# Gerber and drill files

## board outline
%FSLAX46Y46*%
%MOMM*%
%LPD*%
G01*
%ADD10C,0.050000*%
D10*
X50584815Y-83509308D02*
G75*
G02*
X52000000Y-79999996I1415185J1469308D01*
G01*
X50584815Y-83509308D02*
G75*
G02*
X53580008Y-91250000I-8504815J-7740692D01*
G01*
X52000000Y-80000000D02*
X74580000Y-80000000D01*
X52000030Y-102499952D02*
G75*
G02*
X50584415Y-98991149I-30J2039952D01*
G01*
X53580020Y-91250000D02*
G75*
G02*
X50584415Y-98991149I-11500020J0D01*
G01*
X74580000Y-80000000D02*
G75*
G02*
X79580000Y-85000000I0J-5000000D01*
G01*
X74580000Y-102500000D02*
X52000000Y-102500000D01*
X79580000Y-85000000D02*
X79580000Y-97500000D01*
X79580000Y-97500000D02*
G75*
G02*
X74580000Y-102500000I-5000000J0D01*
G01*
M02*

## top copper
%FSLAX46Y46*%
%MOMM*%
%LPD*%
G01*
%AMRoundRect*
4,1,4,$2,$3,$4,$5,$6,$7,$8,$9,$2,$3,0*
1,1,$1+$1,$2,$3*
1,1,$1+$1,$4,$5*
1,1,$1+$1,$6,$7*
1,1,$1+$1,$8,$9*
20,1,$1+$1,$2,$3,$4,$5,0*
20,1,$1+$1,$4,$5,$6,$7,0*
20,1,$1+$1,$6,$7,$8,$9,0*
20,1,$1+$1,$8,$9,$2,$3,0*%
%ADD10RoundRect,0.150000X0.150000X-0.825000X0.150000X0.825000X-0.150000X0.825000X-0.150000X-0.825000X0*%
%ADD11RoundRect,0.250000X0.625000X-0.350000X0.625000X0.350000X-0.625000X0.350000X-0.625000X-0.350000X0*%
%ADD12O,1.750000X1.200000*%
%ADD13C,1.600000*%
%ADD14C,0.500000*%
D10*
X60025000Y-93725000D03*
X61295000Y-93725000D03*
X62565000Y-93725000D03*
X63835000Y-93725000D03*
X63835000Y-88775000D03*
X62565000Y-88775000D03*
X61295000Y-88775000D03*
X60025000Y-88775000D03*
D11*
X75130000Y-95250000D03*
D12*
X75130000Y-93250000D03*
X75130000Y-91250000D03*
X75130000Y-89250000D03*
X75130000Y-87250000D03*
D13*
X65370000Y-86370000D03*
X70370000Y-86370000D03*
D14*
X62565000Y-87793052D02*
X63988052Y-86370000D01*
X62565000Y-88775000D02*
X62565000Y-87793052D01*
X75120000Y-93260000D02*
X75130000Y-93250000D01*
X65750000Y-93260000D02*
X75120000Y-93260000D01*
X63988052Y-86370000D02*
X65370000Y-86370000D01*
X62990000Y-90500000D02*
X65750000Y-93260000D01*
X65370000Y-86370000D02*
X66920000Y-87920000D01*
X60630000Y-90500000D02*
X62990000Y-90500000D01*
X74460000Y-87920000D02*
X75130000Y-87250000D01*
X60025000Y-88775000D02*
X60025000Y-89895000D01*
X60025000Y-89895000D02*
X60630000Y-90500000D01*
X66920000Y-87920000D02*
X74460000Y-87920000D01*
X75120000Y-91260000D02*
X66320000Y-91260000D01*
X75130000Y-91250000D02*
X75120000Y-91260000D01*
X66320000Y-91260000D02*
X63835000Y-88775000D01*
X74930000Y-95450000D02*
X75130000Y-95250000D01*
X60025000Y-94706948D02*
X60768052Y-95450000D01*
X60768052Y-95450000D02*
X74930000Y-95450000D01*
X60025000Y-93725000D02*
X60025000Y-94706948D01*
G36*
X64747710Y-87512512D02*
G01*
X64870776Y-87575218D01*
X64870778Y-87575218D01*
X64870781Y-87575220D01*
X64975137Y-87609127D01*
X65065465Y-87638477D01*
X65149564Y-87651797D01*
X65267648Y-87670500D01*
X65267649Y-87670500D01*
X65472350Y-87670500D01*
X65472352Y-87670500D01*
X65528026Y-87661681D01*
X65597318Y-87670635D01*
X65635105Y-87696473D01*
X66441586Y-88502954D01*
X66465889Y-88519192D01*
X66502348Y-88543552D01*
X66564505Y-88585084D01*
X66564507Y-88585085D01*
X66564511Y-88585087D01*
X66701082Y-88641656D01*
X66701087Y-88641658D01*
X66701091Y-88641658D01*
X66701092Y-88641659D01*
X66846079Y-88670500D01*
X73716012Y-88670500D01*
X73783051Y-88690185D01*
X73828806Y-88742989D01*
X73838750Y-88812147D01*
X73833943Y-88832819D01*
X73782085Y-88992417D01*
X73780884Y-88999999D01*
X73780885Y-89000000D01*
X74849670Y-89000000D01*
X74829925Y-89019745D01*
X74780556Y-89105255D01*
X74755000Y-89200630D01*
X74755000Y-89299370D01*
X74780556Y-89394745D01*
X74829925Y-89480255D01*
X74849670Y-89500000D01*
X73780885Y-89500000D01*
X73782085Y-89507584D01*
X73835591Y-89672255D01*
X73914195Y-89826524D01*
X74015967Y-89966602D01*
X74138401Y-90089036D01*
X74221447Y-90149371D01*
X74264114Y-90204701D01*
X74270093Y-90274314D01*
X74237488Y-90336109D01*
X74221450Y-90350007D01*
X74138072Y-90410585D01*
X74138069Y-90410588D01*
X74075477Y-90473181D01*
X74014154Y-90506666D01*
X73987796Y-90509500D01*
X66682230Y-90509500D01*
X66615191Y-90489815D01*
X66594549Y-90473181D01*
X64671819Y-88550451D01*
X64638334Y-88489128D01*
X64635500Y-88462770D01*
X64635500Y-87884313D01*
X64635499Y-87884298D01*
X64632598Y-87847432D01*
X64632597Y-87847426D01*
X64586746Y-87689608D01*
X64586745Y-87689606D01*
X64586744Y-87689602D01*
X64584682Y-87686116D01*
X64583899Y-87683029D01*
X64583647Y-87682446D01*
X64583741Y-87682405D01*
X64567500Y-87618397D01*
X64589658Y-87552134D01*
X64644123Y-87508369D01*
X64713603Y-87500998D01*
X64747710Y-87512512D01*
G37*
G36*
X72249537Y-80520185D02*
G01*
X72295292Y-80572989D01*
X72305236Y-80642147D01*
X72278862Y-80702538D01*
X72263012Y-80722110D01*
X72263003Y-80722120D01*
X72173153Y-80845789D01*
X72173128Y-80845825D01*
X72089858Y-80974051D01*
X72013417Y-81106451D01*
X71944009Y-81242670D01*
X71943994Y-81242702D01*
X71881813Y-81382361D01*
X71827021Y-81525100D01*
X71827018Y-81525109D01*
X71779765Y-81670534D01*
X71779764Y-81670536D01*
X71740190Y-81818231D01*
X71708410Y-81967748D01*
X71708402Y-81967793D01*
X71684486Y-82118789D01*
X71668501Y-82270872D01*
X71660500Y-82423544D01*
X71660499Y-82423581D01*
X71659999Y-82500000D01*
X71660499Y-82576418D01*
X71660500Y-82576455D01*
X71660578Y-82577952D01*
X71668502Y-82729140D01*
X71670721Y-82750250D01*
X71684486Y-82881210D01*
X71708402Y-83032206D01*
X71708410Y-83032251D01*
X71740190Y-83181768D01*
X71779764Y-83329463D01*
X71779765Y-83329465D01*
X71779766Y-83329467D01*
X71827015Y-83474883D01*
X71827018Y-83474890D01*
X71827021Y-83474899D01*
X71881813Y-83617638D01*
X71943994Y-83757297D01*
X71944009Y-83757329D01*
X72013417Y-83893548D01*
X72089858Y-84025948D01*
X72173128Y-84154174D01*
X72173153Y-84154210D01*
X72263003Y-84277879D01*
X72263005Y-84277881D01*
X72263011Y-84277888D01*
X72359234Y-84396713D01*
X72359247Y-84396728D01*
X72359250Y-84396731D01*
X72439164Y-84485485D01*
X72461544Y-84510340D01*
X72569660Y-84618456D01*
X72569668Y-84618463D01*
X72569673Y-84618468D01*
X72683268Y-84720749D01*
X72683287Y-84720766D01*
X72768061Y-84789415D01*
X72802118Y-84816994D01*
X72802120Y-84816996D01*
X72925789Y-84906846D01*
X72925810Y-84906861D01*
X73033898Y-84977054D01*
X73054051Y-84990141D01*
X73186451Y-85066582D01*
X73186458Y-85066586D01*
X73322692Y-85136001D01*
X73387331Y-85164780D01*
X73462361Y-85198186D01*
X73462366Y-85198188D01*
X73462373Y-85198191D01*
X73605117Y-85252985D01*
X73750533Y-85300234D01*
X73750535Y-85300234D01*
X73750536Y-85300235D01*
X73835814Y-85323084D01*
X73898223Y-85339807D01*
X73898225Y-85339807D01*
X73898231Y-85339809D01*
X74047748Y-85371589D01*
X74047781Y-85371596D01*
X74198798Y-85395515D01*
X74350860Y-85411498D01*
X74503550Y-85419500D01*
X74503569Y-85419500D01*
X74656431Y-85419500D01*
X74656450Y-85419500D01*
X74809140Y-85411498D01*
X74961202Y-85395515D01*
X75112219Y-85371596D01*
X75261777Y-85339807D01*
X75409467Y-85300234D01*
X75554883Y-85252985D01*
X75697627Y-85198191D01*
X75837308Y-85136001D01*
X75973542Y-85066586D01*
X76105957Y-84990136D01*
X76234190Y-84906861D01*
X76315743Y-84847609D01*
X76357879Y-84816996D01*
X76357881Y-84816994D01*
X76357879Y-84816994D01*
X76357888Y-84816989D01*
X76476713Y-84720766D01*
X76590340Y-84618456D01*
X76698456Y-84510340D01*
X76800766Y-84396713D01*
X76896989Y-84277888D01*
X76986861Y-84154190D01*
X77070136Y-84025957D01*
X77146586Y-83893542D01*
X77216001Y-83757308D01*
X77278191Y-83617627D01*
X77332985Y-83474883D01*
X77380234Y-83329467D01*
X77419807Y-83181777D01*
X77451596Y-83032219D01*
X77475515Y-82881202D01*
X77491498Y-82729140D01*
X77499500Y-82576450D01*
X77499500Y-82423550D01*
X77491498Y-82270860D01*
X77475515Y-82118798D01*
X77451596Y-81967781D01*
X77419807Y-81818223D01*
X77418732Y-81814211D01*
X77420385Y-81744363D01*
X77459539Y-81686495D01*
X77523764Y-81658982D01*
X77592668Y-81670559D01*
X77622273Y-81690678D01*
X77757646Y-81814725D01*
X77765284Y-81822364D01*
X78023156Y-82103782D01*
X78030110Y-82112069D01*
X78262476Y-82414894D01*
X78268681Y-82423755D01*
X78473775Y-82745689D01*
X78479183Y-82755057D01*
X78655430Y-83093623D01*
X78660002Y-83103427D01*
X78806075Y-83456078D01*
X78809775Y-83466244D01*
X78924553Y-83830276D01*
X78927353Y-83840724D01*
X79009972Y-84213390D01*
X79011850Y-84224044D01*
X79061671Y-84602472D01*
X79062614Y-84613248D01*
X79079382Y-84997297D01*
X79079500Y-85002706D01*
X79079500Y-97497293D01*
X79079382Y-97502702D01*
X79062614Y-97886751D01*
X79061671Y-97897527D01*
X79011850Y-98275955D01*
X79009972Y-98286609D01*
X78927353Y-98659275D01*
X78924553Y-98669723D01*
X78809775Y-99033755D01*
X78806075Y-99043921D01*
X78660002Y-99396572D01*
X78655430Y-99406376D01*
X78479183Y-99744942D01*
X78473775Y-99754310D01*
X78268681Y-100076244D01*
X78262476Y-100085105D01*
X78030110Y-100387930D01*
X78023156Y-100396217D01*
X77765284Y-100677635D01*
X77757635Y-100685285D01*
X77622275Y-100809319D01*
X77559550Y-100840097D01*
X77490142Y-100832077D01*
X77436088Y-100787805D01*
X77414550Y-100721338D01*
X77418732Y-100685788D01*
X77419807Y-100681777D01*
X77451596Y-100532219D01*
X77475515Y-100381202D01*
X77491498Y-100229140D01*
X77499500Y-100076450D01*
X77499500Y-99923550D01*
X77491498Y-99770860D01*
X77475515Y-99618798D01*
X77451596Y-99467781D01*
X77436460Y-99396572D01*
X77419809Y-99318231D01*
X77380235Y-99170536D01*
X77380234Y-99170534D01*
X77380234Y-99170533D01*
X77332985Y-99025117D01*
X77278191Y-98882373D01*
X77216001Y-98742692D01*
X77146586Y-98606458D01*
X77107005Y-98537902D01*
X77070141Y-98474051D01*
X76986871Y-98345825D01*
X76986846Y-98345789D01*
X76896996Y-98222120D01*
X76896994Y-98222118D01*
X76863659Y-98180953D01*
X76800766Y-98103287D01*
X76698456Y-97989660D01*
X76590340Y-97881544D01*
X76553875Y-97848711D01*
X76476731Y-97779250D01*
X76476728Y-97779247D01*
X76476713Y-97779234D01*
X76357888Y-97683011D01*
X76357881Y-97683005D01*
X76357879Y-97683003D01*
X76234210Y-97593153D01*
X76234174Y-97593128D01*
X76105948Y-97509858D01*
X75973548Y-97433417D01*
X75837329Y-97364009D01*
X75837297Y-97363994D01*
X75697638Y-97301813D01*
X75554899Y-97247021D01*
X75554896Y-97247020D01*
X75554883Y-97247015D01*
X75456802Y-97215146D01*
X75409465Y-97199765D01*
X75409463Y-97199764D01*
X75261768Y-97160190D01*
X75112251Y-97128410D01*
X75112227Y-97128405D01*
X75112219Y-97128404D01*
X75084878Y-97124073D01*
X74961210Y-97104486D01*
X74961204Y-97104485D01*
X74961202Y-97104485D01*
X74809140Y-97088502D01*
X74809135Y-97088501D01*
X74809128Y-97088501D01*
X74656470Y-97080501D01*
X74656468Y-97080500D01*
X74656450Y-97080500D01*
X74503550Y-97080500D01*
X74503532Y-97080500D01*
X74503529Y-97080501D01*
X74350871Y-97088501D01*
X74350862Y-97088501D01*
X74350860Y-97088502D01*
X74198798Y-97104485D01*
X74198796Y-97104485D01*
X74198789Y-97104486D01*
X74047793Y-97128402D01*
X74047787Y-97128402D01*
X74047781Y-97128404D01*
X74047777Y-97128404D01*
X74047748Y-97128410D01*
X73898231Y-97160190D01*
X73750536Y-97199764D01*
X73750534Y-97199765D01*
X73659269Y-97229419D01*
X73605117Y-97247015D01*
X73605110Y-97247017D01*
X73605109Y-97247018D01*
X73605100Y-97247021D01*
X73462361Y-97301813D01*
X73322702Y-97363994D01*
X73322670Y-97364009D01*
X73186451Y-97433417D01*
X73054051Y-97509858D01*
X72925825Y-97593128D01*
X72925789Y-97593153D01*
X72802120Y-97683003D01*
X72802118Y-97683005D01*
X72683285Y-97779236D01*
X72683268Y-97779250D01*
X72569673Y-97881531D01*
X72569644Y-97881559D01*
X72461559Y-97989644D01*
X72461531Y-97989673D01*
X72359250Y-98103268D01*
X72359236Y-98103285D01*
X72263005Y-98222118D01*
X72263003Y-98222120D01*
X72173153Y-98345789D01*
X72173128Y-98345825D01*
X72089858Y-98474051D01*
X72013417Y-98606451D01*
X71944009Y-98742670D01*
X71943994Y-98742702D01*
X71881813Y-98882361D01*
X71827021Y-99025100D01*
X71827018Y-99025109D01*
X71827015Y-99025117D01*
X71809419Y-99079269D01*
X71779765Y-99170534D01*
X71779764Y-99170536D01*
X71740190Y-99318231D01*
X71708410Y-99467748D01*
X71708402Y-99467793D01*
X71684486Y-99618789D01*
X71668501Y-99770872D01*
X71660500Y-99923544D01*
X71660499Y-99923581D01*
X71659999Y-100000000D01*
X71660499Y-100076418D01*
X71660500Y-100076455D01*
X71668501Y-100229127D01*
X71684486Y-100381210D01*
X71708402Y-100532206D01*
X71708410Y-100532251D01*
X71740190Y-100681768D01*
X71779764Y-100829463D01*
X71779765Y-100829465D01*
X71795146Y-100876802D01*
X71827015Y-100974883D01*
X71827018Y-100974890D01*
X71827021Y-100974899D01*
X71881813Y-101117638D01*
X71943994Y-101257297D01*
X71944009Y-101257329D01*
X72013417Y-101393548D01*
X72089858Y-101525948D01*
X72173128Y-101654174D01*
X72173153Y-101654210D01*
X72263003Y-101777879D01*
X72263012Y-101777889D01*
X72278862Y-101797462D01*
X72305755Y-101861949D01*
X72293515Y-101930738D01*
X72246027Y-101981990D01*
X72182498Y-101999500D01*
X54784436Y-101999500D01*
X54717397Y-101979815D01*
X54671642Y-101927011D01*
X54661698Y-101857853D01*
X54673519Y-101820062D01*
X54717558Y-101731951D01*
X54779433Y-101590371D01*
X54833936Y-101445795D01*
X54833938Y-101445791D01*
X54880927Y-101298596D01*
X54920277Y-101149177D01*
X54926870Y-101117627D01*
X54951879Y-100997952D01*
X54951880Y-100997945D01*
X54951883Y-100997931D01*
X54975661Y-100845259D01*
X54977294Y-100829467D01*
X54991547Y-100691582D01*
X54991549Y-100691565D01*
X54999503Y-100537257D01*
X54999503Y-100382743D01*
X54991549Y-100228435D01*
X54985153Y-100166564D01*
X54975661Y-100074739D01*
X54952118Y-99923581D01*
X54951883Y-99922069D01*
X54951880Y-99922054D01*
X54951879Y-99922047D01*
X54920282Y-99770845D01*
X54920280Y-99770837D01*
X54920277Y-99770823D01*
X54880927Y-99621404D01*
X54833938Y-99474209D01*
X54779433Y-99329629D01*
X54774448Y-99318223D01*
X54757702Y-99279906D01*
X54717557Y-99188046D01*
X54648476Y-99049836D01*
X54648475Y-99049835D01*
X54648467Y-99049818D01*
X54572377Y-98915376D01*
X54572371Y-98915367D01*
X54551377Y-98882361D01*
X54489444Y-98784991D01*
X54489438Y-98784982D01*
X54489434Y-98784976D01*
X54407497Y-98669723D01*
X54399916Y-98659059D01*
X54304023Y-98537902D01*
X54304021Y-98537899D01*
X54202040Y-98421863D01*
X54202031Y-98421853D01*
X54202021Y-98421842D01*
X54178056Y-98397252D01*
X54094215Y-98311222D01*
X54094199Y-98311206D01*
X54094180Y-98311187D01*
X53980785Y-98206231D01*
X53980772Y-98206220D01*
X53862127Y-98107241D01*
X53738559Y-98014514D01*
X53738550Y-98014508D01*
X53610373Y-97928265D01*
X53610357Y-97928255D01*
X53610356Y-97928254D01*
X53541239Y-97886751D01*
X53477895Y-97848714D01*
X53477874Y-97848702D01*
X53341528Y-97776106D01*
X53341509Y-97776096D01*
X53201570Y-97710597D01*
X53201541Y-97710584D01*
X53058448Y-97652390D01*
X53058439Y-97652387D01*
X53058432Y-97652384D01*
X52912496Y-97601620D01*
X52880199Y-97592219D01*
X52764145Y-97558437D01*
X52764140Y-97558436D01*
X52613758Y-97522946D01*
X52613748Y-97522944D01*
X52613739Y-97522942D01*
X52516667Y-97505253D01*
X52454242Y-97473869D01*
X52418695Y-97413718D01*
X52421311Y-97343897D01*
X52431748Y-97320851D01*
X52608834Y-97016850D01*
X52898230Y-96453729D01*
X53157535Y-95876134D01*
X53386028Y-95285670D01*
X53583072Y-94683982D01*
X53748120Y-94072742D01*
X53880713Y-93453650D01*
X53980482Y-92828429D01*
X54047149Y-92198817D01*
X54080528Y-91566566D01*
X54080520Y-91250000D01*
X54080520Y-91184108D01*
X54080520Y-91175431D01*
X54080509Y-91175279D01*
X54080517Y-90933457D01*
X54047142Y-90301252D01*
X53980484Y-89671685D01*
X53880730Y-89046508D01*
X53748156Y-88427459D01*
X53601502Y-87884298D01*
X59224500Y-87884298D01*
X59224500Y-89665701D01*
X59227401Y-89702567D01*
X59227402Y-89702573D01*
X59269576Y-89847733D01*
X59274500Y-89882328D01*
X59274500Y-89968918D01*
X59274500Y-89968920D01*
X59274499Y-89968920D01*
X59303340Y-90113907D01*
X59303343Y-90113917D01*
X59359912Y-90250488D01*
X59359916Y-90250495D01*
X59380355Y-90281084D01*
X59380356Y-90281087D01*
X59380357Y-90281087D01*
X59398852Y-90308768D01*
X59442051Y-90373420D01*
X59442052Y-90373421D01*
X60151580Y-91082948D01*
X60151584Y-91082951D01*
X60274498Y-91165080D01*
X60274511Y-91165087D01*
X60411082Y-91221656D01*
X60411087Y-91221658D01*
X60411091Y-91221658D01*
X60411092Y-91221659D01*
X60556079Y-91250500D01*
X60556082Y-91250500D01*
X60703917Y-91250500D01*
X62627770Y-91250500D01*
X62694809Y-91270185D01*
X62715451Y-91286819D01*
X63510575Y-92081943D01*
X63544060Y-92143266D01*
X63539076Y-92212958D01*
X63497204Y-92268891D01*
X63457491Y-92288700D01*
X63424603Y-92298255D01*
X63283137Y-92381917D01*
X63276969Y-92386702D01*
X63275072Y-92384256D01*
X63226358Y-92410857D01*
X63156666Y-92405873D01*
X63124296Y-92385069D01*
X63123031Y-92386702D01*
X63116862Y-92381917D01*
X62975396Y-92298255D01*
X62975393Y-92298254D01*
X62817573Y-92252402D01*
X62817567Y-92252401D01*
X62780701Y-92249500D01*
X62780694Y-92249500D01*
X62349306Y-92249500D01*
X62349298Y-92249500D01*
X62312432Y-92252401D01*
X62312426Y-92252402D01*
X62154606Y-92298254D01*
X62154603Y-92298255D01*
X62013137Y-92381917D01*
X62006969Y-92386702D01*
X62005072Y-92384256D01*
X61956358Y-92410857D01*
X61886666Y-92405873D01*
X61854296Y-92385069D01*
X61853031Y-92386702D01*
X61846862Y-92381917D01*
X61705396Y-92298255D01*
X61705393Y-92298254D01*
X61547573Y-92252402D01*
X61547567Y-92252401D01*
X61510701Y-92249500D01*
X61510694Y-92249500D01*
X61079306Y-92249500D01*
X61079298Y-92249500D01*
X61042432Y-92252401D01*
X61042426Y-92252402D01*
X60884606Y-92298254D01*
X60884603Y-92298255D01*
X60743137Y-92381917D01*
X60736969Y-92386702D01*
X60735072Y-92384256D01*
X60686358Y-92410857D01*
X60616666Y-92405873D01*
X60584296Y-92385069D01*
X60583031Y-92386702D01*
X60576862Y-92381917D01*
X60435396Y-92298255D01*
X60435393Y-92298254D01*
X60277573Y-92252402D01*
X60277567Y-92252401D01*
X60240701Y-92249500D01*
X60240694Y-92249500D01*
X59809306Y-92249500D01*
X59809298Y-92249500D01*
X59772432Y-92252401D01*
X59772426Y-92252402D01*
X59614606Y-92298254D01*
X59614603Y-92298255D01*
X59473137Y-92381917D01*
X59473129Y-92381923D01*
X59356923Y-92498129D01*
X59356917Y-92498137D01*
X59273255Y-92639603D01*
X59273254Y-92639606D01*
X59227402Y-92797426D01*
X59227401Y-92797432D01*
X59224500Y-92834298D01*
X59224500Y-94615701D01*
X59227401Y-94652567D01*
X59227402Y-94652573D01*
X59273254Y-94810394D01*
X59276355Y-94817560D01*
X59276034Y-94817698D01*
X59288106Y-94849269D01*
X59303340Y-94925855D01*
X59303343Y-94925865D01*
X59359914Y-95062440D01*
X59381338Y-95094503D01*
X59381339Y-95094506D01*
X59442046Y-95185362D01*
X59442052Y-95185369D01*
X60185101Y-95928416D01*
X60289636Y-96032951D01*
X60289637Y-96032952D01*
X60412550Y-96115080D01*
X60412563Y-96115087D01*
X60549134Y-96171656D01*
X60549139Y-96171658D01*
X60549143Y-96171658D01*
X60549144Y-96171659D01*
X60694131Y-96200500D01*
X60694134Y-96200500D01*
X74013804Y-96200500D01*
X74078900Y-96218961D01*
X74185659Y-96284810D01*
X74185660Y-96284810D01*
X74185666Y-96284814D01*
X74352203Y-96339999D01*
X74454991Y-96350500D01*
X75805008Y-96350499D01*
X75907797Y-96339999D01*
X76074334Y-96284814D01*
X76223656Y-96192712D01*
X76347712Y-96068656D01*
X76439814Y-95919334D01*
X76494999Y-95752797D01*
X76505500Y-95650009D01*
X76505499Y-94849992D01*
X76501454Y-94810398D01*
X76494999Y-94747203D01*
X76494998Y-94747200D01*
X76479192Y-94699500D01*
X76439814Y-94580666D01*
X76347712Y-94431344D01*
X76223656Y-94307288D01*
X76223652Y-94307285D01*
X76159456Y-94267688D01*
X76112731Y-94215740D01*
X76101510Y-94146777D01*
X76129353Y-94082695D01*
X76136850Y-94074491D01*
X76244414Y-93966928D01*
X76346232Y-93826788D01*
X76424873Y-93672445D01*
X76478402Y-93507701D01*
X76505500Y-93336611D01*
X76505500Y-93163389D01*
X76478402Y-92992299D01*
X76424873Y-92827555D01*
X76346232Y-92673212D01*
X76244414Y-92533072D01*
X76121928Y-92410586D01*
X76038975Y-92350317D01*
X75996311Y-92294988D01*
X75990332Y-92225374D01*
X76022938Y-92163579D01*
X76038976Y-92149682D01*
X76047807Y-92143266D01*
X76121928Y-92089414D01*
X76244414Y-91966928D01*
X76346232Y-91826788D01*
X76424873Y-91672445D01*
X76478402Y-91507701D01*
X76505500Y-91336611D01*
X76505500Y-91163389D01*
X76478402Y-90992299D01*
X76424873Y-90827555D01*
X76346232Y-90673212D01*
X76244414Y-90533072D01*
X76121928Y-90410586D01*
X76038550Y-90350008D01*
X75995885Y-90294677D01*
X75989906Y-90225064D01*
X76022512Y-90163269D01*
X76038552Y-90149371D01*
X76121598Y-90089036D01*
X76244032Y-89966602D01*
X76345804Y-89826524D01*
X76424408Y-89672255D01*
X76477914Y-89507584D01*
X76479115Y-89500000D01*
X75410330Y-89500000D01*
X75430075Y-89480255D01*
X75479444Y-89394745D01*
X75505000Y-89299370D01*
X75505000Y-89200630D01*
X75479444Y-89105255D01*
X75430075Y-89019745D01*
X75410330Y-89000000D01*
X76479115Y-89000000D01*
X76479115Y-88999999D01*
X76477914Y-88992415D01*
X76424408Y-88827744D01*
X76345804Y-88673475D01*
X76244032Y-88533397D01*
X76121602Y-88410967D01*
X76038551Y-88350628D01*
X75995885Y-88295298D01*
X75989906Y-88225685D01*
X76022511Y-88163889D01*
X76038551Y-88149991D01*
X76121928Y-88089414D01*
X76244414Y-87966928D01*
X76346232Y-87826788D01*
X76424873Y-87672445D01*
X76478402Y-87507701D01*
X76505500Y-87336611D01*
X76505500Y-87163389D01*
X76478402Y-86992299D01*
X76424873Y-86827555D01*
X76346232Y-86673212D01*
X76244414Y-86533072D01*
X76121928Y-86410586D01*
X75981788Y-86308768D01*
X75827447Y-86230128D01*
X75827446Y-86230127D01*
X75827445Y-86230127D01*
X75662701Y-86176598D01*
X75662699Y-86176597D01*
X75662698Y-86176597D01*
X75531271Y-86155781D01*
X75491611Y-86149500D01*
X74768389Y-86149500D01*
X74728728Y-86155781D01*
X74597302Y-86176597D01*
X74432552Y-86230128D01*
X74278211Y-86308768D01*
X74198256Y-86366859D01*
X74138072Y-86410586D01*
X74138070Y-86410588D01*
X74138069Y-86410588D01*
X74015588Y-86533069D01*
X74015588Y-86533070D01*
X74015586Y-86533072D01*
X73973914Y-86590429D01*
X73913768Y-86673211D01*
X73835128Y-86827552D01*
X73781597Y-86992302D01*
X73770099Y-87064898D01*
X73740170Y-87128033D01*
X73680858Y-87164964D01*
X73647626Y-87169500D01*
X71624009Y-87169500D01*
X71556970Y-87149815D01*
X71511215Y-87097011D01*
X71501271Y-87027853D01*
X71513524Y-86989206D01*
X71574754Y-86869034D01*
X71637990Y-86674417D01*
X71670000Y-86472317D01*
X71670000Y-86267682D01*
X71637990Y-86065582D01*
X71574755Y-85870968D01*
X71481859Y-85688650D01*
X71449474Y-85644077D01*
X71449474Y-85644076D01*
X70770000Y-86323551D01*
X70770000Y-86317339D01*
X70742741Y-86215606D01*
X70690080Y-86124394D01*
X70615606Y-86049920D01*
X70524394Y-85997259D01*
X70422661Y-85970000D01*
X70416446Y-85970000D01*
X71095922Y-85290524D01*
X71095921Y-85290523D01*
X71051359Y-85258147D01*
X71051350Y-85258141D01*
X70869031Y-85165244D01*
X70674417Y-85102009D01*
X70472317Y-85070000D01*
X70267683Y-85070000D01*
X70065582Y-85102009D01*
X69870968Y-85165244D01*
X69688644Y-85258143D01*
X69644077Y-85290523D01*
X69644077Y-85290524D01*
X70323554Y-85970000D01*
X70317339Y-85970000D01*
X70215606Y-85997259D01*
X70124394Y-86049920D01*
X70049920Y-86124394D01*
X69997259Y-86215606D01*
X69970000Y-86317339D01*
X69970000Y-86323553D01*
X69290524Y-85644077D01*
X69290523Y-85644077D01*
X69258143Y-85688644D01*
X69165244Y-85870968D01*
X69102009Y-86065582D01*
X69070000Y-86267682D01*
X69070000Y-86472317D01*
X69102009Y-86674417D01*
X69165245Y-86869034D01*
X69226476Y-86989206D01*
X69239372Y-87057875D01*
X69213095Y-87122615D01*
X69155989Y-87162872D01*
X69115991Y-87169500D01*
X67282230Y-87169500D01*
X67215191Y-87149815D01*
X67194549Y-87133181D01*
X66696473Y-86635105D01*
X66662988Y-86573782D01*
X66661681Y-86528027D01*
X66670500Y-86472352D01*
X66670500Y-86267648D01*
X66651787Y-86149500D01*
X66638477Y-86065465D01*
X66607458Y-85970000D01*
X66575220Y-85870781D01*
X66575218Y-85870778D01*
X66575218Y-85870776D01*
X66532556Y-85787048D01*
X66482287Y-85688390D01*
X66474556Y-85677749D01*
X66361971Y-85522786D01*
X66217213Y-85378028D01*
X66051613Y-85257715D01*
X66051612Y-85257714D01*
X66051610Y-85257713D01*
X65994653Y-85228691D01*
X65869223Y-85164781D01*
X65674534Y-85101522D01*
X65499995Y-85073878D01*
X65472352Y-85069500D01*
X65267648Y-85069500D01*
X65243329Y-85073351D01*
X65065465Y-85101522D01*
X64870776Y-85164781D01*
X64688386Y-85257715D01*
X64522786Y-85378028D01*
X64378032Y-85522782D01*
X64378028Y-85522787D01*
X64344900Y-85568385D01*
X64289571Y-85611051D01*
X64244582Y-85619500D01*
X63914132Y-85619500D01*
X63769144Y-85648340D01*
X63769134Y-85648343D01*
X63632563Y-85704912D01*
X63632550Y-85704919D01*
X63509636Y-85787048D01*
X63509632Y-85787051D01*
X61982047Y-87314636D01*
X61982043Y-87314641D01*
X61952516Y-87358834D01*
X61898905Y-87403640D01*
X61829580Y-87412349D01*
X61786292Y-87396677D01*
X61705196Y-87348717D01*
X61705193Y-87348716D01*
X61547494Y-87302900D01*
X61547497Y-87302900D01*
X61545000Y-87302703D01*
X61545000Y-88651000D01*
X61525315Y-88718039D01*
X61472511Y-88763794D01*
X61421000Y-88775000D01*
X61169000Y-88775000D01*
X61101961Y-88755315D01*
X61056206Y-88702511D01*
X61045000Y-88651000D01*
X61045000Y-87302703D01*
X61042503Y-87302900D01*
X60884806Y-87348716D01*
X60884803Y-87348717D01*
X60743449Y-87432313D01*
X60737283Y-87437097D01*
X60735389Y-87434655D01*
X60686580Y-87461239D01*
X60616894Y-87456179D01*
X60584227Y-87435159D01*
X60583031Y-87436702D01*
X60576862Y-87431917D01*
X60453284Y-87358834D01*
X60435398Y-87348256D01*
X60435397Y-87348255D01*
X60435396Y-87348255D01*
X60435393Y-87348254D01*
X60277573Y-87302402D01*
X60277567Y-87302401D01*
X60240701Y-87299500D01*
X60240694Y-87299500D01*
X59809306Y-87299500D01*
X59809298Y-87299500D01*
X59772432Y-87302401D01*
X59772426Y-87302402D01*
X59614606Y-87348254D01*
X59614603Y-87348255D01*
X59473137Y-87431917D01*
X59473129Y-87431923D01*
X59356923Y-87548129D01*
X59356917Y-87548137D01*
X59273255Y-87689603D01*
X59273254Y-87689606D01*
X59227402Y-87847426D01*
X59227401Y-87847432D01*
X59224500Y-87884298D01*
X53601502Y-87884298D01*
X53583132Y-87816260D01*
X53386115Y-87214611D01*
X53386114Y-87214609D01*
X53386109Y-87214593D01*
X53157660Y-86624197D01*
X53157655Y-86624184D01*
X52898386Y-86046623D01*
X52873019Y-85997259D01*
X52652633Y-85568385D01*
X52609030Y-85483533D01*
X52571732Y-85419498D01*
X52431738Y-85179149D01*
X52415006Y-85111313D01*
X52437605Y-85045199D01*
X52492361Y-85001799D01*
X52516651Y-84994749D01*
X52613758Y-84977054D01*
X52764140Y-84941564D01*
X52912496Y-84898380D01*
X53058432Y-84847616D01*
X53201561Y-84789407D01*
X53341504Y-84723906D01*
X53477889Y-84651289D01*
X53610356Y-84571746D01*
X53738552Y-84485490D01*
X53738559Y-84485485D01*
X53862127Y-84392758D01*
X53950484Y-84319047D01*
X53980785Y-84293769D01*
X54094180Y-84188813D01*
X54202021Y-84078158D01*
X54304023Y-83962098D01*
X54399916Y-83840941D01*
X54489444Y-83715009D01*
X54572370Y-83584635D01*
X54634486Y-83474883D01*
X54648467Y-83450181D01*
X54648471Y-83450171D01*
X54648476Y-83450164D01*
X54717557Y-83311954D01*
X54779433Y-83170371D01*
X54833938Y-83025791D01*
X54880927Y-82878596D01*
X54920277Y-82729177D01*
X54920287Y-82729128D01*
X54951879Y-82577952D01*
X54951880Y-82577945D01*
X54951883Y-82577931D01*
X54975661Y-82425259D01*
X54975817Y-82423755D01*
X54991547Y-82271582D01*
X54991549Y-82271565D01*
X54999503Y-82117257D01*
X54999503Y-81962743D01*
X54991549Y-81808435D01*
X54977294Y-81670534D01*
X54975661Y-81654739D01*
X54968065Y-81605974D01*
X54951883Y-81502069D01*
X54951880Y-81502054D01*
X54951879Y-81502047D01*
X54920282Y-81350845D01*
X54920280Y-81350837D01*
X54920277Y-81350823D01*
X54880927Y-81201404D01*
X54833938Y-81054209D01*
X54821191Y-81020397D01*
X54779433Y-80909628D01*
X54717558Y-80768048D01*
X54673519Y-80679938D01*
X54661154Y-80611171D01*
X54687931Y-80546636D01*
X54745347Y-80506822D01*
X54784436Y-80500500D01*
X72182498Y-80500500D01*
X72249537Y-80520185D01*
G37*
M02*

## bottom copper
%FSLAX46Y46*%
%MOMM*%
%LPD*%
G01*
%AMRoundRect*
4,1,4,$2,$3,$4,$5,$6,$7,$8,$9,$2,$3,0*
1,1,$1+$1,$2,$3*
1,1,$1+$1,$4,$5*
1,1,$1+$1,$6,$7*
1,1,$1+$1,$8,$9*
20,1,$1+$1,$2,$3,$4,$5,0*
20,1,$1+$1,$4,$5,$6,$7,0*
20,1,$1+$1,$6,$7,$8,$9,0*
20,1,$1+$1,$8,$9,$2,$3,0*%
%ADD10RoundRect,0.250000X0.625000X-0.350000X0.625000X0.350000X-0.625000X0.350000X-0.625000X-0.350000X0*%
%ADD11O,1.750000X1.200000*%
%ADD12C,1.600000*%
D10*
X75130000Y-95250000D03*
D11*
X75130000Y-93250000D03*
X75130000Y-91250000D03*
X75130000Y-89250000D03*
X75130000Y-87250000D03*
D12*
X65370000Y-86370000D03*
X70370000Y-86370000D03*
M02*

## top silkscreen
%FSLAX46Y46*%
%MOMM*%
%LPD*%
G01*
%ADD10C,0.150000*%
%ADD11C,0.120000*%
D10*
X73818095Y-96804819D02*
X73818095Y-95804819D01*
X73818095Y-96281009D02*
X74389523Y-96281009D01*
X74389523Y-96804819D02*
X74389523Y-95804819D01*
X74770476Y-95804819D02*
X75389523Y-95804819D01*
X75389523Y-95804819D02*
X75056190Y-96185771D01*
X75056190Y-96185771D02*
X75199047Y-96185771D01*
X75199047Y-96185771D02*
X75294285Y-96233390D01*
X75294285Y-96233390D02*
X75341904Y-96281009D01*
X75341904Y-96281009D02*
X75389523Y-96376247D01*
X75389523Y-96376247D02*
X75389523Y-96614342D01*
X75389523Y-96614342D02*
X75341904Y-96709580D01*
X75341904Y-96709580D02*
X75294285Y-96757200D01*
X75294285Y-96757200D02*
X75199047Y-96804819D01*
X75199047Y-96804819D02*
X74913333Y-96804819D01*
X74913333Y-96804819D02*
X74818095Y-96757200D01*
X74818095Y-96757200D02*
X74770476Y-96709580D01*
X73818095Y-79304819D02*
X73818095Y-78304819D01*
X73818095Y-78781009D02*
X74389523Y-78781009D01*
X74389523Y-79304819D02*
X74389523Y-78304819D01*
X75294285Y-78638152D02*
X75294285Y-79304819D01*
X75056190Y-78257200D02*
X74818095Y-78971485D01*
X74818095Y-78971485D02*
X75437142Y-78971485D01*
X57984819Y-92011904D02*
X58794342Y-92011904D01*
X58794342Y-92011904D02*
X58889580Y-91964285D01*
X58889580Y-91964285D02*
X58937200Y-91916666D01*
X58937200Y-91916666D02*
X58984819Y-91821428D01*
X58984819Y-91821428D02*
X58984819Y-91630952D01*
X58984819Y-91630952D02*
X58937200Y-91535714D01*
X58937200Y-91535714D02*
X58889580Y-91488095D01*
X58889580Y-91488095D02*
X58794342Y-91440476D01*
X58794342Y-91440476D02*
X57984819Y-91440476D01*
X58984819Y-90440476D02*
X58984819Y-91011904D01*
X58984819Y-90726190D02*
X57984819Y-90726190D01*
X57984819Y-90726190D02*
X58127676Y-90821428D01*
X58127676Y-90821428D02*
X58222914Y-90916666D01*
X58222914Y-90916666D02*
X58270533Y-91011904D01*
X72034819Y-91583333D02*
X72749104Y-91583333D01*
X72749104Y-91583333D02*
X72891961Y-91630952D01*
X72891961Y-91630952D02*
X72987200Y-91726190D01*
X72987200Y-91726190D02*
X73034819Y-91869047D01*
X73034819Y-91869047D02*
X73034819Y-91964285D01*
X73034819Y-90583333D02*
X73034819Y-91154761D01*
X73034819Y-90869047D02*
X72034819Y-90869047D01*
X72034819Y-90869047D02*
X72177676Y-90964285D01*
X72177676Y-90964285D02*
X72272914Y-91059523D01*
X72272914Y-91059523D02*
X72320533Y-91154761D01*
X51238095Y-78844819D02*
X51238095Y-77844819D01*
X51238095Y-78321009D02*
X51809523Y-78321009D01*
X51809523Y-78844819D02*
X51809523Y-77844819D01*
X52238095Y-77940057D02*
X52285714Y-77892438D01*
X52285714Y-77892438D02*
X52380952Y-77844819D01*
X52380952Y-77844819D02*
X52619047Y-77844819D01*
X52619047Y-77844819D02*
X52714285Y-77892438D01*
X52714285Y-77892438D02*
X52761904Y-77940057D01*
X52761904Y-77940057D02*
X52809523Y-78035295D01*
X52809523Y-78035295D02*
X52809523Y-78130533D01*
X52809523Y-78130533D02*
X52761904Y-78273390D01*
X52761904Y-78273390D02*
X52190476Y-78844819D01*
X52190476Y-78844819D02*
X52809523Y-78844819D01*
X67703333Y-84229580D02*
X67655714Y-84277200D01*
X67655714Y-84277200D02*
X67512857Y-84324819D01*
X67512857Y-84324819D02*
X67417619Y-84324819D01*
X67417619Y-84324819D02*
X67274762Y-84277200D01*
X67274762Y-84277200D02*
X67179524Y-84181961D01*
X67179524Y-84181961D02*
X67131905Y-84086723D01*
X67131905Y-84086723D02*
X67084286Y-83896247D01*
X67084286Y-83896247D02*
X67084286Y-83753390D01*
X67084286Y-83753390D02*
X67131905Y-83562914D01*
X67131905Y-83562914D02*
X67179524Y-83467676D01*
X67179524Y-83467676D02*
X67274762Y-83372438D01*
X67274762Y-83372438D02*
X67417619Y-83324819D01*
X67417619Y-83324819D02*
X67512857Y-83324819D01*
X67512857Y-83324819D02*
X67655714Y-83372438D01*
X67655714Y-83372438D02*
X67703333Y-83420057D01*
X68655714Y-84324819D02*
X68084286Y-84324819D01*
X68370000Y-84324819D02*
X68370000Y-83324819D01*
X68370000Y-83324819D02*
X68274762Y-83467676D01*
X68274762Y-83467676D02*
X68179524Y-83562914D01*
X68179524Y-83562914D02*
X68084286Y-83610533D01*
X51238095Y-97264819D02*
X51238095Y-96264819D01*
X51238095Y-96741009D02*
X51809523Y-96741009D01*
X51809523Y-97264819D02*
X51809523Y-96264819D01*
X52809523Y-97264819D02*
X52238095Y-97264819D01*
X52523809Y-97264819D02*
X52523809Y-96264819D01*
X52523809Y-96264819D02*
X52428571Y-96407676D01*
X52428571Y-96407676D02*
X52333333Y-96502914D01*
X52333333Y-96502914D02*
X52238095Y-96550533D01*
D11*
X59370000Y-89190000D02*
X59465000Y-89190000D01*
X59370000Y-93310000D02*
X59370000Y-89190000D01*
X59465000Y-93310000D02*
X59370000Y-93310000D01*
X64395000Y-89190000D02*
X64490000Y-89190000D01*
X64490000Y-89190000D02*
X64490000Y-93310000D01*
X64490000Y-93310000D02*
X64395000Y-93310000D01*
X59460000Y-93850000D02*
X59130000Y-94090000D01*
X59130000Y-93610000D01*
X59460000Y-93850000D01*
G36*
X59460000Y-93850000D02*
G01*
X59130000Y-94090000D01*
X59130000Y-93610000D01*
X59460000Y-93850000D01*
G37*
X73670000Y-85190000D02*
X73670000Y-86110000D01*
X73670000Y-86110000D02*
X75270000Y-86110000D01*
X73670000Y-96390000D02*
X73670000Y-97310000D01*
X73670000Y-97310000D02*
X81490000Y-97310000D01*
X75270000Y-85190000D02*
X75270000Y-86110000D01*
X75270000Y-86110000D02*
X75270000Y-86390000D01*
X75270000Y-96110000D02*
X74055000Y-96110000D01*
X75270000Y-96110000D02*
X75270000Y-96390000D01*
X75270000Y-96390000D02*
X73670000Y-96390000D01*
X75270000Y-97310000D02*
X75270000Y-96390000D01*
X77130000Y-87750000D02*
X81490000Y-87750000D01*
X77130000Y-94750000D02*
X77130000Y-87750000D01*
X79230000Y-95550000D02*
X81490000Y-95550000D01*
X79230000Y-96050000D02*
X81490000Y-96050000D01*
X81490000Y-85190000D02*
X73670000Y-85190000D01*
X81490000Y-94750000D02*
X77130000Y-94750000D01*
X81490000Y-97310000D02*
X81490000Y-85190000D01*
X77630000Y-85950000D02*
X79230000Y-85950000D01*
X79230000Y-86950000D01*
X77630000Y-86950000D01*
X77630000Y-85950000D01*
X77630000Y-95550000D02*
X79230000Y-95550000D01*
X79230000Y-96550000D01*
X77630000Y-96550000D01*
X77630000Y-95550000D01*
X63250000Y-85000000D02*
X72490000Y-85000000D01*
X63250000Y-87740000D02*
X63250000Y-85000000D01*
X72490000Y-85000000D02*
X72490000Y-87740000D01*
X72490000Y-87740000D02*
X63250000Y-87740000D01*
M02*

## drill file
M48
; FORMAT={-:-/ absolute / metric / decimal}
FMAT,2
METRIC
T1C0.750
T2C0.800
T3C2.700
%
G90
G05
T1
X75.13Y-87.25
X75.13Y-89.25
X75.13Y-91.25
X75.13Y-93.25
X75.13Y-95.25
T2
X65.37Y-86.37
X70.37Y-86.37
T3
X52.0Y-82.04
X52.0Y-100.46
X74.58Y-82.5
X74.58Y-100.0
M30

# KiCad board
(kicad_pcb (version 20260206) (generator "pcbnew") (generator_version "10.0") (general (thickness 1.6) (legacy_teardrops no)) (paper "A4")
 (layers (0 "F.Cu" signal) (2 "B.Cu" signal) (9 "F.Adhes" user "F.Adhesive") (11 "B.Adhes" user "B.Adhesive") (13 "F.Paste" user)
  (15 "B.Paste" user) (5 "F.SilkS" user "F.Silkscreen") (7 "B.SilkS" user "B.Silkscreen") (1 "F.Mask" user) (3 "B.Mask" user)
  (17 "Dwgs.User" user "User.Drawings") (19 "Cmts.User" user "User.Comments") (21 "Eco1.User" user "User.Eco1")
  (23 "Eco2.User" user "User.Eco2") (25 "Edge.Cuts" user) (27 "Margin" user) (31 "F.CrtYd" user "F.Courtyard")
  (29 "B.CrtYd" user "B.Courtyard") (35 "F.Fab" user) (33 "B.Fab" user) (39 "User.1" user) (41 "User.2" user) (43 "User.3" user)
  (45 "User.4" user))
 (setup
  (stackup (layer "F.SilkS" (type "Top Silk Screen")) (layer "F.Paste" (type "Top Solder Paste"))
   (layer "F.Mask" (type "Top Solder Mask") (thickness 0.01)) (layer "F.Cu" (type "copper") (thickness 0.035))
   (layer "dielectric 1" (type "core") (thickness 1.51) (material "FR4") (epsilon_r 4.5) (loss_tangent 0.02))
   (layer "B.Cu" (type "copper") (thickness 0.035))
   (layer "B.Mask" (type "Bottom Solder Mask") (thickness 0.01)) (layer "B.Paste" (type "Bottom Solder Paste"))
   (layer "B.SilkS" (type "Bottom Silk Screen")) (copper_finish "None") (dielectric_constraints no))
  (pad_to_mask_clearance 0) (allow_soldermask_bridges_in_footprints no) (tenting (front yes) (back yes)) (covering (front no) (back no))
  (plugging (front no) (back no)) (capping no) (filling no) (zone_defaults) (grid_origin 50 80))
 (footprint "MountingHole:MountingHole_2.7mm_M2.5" (layer "F.Cu") (at 74.58 100)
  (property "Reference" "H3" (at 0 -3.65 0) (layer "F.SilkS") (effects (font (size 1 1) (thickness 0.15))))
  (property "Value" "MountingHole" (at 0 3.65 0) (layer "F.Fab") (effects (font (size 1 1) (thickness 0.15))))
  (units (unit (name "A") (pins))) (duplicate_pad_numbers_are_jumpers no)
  (pad "" np_thru_hole circle (at 0 0) (size 2.7 2.7) (drill 2.7) (layers "*.Cu" "*.Mask")))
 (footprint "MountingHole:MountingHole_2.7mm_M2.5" (layer "F.Cu") (at 74.58 82.5)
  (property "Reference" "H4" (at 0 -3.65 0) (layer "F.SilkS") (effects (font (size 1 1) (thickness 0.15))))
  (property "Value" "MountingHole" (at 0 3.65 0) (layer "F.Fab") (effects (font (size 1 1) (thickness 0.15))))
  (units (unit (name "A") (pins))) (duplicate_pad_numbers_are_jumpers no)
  (pad "" np_thru_hole circle (at 0 0) (size 2.7 2.7) (drill 2.7) (layers "*.Cu" "*.Mask")))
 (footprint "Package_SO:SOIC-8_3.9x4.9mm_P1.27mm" (layer "F.Cu") (at 61.93 91.25 90)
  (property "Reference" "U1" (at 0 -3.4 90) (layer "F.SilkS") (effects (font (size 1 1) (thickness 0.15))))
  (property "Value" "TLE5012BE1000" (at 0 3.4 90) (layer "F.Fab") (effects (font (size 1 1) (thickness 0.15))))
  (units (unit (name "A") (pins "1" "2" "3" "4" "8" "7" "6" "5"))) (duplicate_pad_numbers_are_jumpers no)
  (fp_line (start 2.06 -2.56) (end 2.06 -2.465) (stroke (width 0.12) (type solid)) (layer "F.SilkS"))
  (fp_line (start -2.06 -2.56) (end 2.06 -2.56) (stroke (width 0.12) (type solid)) (layer "F.SilkS"))
  (fp_line (start -2.06 -2.465) (end -2.06 -2.56) (stroke (width 0.12) (type solid)) (layer "F.SilkS"))
  (fp_line (start 2.06 2.465) (end 2.06 2.56) (stroke (width 0.12) (type solid)) (layer "F.SilkS"))
  (fp_line (start 2.06 2.56) (end -2.06 2.56) (stroke (width 0.12) (type solid)) (layer "F.SilkS"))
  (fp_line (start -2.06 2.56) (end -2.06 2.465) (stroke (width 0.12) (type solid)) (layer "F.SilkS"))
  (fp_poly (pts (xy -2.6 -2.47) (xy -2.84 -2.8) (xy -2.36 -2.8)) (stroke (width 0.12) (type solid)) (fill yes) (layer "F.SilkS"))
  (pad "1" smd roundrect (at -2.475 -1.905 90) (size 1.95 0.6) (layers "F.Cu" "F.Mask" "F.Paste") (roundrect_rratio 0.25) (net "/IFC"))
  (pad "2" smd roundrect (at -2.475 -0.635 90) (size 1.95 0.6) (layers "F.Cu" "F.Mask" "F.Paste") (roundrect_rratio 0.25)
   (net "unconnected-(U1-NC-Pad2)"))
  (pad "3" smd roundrect (at -2.475 0.635 90) (size 1.95 0.6) (layers "F.Cu" "F.Mask" "F.Paste") (roundrect_rratio 0.25)
   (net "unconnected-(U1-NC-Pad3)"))
  (pad "4" smd roundrect (at -2.475 1.905 90) (size 1.95 0.6) (layers "F.Cu" "F.Mask" "F.Paste") (roundrect_rratio 0.25)
   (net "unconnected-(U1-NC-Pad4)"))
  (pad "5" smd roundrect (at 2.475 1.905 90) (size 1.95 0.6) (layers "F.Cu" "F.Mask" "F.Paste") (roundrect_rratio 0.25) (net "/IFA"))
  (pad "6" smd roundrect (at 2.475 0.635 90) (size 1.95 0.6) (layers "F.Cu" "F.Mask" "F.Paste") (roundrect_rratio 0.25) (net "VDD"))
  (pad "7" smd roundrect (at 2.475 -0.635 90) (size 1.95 0.6) (layers "F.Cu" "F.Mask" "F.Paste") (roundrect_rratio 0.25) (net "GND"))
  (pad "8" smd roundrect (at 2.475 -1.905 90) (size 1.95 0.6) (layers "F.Cu" "F.Mask" "F.Paste") (roundrect_rratio 0.25) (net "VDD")))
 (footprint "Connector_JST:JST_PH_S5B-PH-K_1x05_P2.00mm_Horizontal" (layer "F.Cu") (at 75.13 95.25 90)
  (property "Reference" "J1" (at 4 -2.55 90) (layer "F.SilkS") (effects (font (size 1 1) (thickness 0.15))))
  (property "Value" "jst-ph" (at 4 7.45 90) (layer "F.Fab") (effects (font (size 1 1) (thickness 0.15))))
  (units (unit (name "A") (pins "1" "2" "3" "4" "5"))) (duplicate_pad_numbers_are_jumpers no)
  (fp_line (start 10.06 -1.46) (end 9.14 -1.46) (stroke (width 0.12) (type solid)) (layer "F.SilkS"))
  (fp_line (start 9.14 -1.46) (end 9.14 0.14) (stroke (width 0.12) (type solid)) (layer "F.SilkS"))
  (fp_line (start -1.14 -1.46) (end -2.06 -1.46) (stroke (width 0.12) (type solid)) (layer "F.SilkS"))
  (fp_line (start -2.06 -1.46) (end -2.06 6.36) (stroke (width 0.12) (type solid)) (layer "F.SilkS"))
  (fp_line (start 10.06 0.14) (end 9.14 0.14) (stroke (width 0.12) (type solid)) (layer "F.SilkS"))
  (fp_line (start 9.14 0.14) (end 8.86 0.14) (stroke (width 0.12) (type solid)) (layer "F.SilkS"))
  (fp_line (start -0.86 0.14) (end -0.86 -1.075) (stroke (width 0.12) (type solid)) (layer "F.SilkS"))
  (fp_line (start -0.86 0.14) (end -1.14 0.14) (stroke (width 0.12) (type solid)) (layer "F.SilkS"))
  (fp_line (start -1.14 0.14) (end -1.14 -1.46) (stroke (width 0.12) (type solid)) (layer "F.SilkS"))
  (fp_line (start -2.06 0.14) (end -1.14 0.14) (stroke (width 0.12) (type solid)) (layer "F.SilkS"))
  (fp_line (start 7.5 2) (end 7.5 6.36) (stroke (width 0.12) (type solid)) (layer "F.SilkS"))
  (fp_line (start 0.5 2) (end 7.5 2) (stroke (width 0.12) (type solid)) (layer "F.SilkS"))
  (fp_line (start -0.3 4.1) (end -0.3 6.36) (stroke (width 0.12) (type solid)) (layer "F.SilkS"))
  (fp_line (start -0.8 4.1) (end -0.8 6.36) (stroke (width 0.12) (type solid)) (layer "F.SilkS"))
  (fp_line (start 10.06 6.36) (end 10.06 -1.46) (stroke (width 0.12) (type solid)) (layer "F.SilkS"))
  (fp_line (start 0.5 6.36) (end 0.5 2) (stroke (width 0.12) (type solid)) (layer "F.SilkS"))
  (fp_line (start -2.06 6.36) (end 10.06 6.36) (stroke (width 0.12) (type solid)) (layer "F.SilkS"))
  (fp_rect (start 8.3 2.5) (end 9.3 4.1) (stroke (width 0.12) (type solid)) (fill no) (layer "F.SilkS"))
  (fp_rect (start -1.3 2.5) (end -0.3 4.1) (stroke (width 0.12) (type solid)) (fill no) (layer "F.SilkS"))
  (pad "1" thru_hole roundrect (at 0 0 90) (size 1.2 1.75) (drill 0.75) (layers "*.Cu" "*.Mask") (remove_unused_layers no)
   (roundrect_rratio 0.208333) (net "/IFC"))
  (pad "2" thru_hole oval (at 2 0 90) (size 1.2 1.75) (drill 0.75) (layers "*.Cu" "*.Mask") (remove_unused_layers no) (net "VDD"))
  (pad "3" thru_hole oval (at 4 0 90) (size 1.2 1.75) (drill 0.75) (layers "*.Cu" "*.Mask") (remove_unused_layers no) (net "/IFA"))
  (pad "4" thru_hole oval (at 6 0 90) (size 1.2 1.75) (drill 0.75) (layers "*.Cu" "*.Mask") (remove_unused_layers no) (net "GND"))
  (pad "5" thru_hole oval (at 8 0 90) (size 1.2 1.75) (drill 0.75) (layers "*.Cu" "*.Mask") (remove_unused_layers no) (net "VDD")))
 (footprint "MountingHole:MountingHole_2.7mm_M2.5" (layer "F.Cu") (at 52 82.04)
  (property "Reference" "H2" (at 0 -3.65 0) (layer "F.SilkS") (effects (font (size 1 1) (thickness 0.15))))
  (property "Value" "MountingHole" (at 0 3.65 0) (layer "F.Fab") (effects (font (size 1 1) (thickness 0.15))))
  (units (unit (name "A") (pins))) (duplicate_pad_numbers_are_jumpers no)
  (pad "" np_thru_hole circle (at 0 0) (size 2.7 2.7) (drill 2.7) (layers "*.Cu" "*.Mask")))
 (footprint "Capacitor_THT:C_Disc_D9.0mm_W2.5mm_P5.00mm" (layer "F.Cu") (at 65.37 86.37)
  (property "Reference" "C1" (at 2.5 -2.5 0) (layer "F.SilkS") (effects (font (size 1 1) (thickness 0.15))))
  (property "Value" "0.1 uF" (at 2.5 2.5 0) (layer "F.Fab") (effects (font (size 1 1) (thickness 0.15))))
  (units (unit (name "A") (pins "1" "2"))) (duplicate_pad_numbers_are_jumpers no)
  (fp_line (start -2.12 -1.37) (end 7.12 -1.37) (stroke (width 0.12) (type solid)) (layer "F.SilkS"))
  (fp_line (start -2.12 1.37) (end -2.12 -1.37) (stroke (width 0.12) (type solid)) (layer "F.SilkS"))
  (fp_line (start 7.12 -1.37) (end 7.12 1.37) (stroke (width 0.12) (type solid)) (layer "F.SilkS"))
  (fp_line (start 7.12 1.37) (end -2.12 1.37) (stroke (width 0.12) (type solid)) (layer "F.SilkS"))
  (pad "1" thru_hole circle (at 0 0) (size 1.6 1.6) (drill 0.8) (layers "*.Cu" "*.Mask") (remove_unused_layers no) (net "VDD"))
  (pad "2" thru_hole circle (at 5 0) (size 1.6 1.6) (drill 0.8) (layers "*.Cu" "*.Mask") (remove_unused_layers no) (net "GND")))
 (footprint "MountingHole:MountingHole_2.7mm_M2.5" (layer "F.Cu") (at 52 100.46)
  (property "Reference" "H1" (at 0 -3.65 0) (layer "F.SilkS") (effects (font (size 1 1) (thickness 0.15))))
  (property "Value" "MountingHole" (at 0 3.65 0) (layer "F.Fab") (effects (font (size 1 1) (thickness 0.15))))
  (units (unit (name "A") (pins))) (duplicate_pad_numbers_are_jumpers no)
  (pad "" np_thru_hole circle (at 0 0) (size 2.7 2.7) (drill 2.7) (layers "*.Cu" "*.Mask")))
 (gr_arc (start 50.584815 83.509308) (mid 50.108042 81.277038) (end 52 79.999996) (stroke (width 0.05) (type default)) (layer "Edge.Cuts"))
 (gr_arc (start 50.584815 83.509308) (mid 52.805102 87.100015) (end 53.580008 91.25) (stroke (width 0.05) (type default))
  (layer "Edge.Cuts"))
 (gr_line (start 52 80) (end 74.58 80) (stroke (width 0.05) (type default)) (layer "Edge.Cuts"))
 (gr_arc (start 52.00003 102.499952) (mid 50.108209 101.223237) (end 50.584415 98.991149) (stroke (width 0.05) (type default))
  (layer "Edge.Cuts"))
 (gr_arc (start 53.58002 91.25) (mid 52.805004 95.400272) (end 50.584415 98.991149) (stroke (width 0.05) (type default)) (layer "Edge.Cuts"))
 (gr_arc (start 74.58 80) (mid 78.115534 81.464466) (end 79.58 85) (stroke (width 0.05) (type default)) (layer "Edge.Cuts"))
 (gr_line (start 74.58 102.5) (end 52 102.5) (stroke (width 0.05) (type default)) (layer "Edge.Cuts"))
 (gr_line (start 79.58 85) (end 79.58 97.5) (stroke (width 0.05) (type default)) (layer "Edge.Cuts"))
 (gr_arc (start 79.58 97.5) (mid 78.115534 101.035534) (end 74.58 102.5) (stroke (width 0.05) (type default)) (layer "Edge.Cuts"))
 (segment (start 62.565 87.793052) (end 63.988052 86.37) (width 0.5) (layer "F.Cu") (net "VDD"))
 (segment (start 62.565 88.775) (end 62.565 87.793052) (width 0.5) (layer "F.Cu") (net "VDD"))
 (segment (start 75.12 93.26) (end 75.13 93.25) (width 0.5) (layer "F.Cu") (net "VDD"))
 (segment (start 65.75 93.26) (end 75.12 93.26) (width 0.5) (layer "F.Cu") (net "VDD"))
 (segment (start 63.988052 86.37) (end 65.37 86.37) (width 0.5) (layer "F.Cu") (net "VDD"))
 (segment (start 62.99 90.5) (end 65.75 93.26) (width 0.5) (layer "F.Cu") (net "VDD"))
 (segment (start 65.37 86.37) (end 66.92 87.92) (width 0.5) (layer "F.Cu") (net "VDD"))
 (segment (start 60.63 90.5) (end 62.99 90.5) (width 0.5) (layer "F.Cu") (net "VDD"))
 (segment (start 74.46 87.92) (end 75.13 87.25) (width 0.5) (layer "F.Cu") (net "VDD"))
 (segment (start 60.025 88.775) (end 60.025 89.895) (width 0.5) (layer "F.Cu") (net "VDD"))
 (segment (start 60.025 89.895) (end 60.63 90.5) (width 0.5) (layer "F.Cu") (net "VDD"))
 (segment (start 66.92 87.92) (end 74.46 87.92) (width 0.5) (layer "F.Cu") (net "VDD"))
 (segment (start 75.12 91.26) (end 66.32 91.26) (width 0.5) (layer "F.Cu") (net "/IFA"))
 (segment (start 75.13 91.25) (end 75.12 91.26) (width 0.5) (layer "F.Cu") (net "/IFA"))
 (segment (start 66.32 91.26) (end 63.835 88.775) (width 0.5) (layer "F.Cu") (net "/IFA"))
 (segment (start 74.93 95.45) (end 75.13 95.25) (width 0.5) (layer "F.Cu") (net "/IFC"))
 (segment (start 60.025 94.706948) (end 60.768052 95.45) (width 0.5) (layer "F.Cu") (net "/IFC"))
 (segment (start 60.768052 95.45) (end 74.93 95.45) (width 0.5) (layer "F.Cu") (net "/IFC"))
 (segment (start 60.025 93.725) (end 60.025 94.706948) (width 0.5) (layer "F.Cu") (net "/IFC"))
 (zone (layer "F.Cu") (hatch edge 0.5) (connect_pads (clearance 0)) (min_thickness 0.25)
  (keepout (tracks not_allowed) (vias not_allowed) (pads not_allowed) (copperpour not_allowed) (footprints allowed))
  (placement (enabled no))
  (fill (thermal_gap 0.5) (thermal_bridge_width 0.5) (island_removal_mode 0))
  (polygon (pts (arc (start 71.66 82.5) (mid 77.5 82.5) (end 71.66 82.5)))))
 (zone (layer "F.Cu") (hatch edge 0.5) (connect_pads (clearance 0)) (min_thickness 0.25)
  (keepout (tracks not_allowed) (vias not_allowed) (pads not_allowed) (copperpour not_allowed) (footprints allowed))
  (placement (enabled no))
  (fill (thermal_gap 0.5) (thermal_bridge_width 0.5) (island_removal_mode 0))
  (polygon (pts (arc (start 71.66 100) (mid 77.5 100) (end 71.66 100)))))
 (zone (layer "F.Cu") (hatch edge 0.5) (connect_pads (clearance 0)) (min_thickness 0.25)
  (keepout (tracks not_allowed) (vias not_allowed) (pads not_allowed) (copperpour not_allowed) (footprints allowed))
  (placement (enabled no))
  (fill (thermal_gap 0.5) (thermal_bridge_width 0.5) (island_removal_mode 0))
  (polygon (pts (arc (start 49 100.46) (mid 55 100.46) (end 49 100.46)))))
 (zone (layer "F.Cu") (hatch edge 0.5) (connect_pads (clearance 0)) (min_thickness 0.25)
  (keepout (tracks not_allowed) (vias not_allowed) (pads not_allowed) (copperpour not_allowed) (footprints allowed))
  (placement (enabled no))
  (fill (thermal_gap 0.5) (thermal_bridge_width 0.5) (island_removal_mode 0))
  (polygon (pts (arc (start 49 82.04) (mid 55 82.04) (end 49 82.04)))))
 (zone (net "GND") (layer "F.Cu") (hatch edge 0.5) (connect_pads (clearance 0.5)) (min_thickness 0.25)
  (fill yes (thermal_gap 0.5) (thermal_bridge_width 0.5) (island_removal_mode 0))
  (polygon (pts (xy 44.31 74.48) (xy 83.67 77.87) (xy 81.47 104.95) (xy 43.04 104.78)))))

